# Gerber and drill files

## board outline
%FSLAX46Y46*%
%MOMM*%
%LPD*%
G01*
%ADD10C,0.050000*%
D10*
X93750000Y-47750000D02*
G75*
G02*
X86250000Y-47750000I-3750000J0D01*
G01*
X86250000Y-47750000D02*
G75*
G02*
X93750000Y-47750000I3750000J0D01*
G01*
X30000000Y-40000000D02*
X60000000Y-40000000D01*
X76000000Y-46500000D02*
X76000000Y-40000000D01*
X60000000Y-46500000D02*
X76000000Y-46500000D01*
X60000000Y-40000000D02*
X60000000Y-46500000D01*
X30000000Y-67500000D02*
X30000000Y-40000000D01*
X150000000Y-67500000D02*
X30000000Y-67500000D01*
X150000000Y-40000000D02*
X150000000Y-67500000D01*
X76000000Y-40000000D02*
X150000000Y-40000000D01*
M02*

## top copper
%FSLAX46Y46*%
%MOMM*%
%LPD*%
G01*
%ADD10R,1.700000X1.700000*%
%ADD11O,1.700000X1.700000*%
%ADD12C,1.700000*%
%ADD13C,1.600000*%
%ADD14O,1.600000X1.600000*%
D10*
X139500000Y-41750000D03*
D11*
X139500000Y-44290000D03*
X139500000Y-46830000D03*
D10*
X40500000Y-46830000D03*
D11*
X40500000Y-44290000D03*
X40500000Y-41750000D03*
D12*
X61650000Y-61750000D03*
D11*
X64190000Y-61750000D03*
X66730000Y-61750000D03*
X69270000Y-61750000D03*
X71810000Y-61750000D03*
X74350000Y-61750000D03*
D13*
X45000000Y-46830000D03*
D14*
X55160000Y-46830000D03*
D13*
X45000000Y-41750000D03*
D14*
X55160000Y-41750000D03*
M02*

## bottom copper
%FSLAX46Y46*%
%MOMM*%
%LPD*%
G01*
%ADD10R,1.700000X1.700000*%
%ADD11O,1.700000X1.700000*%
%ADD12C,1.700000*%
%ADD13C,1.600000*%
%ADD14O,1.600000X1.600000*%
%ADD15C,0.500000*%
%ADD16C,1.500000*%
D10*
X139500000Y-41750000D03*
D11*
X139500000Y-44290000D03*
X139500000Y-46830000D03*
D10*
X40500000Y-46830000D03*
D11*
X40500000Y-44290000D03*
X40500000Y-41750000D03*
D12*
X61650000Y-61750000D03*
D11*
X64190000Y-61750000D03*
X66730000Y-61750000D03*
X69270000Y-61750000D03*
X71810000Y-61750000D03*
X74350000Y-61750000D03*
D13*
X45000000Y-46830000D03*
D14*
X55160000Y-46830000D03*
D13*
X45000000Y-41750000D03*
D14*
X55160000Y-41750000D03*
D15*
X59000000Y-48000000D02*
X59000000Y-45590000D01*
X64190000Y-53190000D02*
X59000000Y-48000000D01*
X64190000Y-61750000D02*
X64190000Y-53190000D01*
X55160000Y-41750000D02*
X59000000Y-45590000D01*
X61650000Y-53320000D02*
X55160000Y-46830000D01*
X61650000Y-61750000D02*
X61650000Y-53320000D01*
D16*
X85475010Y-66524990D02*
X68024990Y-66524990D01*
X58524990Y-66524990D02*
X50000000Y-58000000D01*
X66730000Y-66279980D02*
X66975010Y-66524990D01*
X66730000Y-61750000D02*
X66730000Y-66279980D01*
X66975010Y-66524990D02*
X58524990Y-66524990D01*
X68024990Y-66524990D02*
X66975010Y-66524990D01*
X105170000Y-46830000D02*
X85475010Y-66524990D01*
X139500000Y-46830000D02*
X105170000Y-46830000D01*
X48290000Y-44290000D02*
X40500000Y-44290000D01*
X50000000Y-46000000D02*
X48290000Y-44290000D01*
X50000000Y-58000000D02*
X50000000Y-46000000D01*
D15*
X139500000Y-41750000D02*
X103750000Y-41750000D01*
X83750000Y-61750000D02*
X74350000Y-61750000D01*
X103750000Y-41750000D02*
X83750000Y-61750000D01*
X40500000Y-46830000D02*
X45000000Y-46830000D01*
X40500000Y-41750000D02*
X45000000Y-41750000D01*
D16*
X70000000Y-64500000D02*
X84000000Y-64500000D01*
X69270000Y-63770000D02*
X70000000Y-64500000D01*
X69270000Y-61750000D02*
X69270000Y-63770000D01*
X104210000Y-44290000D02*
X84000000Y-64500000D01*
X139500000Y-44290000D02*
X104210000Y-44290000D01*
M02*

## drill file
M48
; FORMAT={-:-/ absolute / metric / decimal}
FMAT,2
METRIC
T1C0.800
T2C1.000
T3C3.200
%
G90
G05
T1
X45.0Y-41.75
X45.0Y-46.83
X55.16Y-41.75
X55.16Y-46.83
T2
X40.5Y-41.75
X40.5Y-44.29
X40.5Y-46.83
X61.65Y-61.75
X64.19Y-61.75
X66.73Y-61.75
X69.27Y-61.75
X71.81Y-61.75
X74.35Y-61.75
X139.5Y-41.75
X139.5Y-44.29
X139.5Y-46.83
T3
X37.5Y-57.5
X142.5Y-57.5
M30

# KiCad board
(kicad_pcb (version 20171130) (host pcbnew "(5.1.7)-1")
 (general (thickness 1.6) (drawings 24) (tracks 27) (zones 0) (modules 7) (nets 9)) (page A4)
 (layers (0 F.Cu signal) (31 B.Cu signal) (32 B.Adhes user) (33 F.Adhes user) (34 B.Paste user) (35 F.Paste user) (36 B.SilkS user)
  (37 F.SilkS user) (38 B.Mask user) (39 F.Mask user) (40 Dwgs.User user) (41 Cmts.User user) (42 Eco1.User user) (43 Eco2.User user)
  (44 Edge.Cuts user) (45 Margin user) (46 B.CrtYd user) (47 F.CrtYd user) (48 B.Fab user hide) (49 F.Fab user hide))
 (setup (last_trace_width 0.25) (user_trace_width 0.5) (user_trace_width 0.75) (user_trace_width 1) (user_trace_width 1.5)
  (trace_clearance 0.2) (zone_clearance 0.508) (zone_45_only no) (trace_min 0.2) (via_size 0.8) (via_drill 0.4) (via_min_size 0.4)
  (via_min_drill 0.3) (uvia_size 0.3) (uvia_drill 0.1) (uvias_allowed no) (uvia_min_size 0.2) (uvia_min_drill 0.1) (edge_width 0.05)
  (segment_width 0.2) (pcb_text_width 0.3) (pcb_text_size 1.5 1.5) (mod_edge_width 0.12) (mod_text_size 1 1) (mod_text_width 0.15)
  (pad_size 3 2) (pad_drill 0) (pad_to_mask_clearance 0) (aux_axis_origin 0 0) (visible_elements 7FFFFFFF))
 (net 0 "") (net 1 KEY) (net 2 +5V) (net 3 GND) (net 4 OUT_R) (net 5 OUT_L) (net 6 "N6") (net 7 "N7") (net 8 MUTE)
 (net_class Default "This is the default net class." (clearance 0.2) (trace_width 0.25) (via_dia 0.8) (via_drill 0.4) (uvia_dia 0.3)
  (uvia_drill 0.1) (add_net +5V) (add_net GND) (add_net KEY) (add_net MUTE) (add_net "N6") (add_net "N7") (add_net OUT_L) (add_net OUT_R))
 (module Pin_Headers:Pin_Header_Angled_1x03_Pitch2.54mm (layer F.Cu) (at 139.5 41.75)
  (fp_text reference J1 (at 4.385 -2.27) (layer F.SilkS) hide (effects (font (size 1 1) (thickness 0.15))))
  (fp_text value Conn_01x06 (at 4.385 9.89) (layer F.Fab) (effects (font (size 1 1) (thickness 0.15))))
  (pad 1 thru_hole rect (at 0 0) (size 1.7 1.7) (drill 1) (layers *.Cu *.Mask) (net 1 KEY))
  (pad 2 thru_hole oval (at 0 2.54) (size 1.7 1.7) (drill 1) (layers *.Cu *.Mask) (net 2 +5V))
  (pad 3 thru_hole oval (at 0 5.08) (size 1.7 1.7) (drill 1) (layers *.Cu *.Mask) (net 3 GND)))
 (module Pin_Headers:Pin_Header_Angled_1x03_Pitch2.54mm (layer F.Cu) (at 40.5 46.83 180)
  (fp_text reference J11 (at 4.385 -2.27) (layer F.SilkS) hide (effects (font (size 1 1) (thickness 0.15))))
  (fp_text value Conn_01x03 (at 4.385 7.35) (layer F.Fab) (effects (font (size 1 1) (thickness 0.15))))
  (pad 1 thru_hole rect (at 0 0 180) (size 1.7 1.7) (drill 1) (layers *.Cu *.Mask) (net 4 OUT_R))
  (pad 2 thru_hole oval (at 0 2.54 180) (size 1.7 1.7) (drill 1) (layers *.Cu *.Mask) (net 3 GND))
  (pad 3 thru_hole oval (at 0 5.08 180) (size 1.7 1.7) (drill 1) (layers *.Cu *.Mask) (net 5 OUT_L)))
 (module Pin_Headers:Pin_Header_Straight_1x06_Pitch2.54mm (layer F.Cu) (at 61.65 61.75 90)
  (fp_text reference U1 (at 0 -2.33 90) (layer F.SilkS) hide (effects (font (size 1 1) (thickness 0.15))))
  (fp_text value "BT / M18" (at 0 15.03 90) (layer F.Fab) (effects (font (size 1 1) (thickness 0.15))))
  (pad 1 thru_hole circle (at 0 0 90) (size 1.7 1.7) (drill 1) (layers *.Cu *.Mask) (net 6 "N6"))
  (pad 2 thru_hole oval (at 0 2.54 90) (size 1.7 1.7) (drill 1) (layers *.Cu *.Mask) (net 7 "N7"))
  (pad 3 thru_hole oval (at 0 5.08 90) (size 1.7 1.7) (drill 1) (layers *.Cu *.Mask) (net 3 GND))
  (pad 4 thru_hole oval (at 0 7.62 90) (size 1.7 1.7) (drill 1) (layers *.Cu *.Mask) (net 2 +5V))
  (pad 5 thru_hole oval (at 0 10.16 90) (size 1.7 1.7) (drill 1) (layers *.Cu *.Mask) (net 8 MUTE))
  (pad 6 thru_hole oval (at 0 12.7 90) (size 1.7 1.7) (drill 1) (layers *.Cu *.Mask) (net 1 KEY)))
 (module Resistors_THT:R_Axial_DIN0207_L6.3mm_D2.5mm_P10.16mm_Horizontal (layer F.Cu) (at 45 46.83)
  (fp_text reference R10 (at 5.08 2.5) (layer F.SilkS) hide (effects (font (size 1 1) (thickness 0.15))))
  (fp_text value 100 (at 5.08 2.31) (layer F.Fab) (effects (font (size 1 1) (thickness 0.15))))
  (pad 1 thru_hole circle (at 0 0) (size 1.6 1.6) (drill 0.8) (layers *.Cu *.Mask) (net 4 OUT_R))
  (pad 2 thru_hole oval (at 10.16 0) (size 1.6 1.6) (drill 0.8) (layers *.Cu *.Mask) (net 6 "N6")))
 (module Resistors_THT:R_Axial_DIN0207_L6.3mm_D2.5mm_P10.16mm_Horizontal (layer F.Cu) (at 45 41.75)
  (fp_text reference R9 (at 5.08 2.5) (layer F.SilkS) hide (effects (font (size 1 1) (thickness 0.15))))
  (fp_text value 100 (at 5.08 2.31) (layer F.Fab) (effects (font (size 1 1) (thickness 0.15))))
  (pad 1 thru_hole circle (at 0 0) (size 1.6 1.6) (drill 0.8) (layers *.Cu *.Mask) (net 5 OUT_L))
  (pad 2 thru_hole oval (at 10.16 0) (size 1.6 1.6) (drill 0.8) (layers *.Cu *.Mask) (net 7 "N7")))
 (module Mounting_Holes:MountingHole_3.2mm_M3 (layer F.Cu) (at 142.5 57.5)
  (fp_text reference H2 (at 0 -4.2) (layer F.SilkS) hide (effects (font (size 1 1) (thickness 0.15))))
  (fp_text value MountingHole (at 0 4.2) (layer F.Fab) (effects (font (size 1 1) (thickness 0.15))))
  (pad 1 np_thru_hole circle (at 0 0) (size 3.2 3.2) (drill 3.2) (layers *.Cu *.Mask)))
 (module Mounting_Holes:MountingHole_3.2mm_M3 (layer F.Cu) (at 37.5 57.5)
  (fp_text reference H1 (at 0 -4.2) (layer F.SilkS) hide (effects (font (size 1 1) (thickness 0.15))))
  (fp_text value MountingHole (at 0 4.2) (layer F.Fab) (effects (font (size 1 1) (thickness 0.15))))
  (pad 1 np_thru_hole circle (at 0 0) (size 3.2 3.2) (drill 3.2) (layers *.Cu *.Mask)))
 (gr_circle (center 90 47.75) (end 93.75 47.75) (layer Edge.Cuts) (width 0.05))
 (gr_line (start 30 40) (end 60 40) (layer Edge.Cuts) (width 0.05))
 (gr_line (start 76 46.5) (end 76 40) (layer Edge.Cuts) (width 0.05))
 (gr_line (start 60 46.5) (end 76 46.5) (layer Edge.Cuts) (width 0.05))
 (gr_line (start 60 40) (end 60 46.5) (layer Edge.Cuts) (width 0.05))
 (gr_line (start 30 67.5) (end 30 40) (layer Edge.Cuts) (width 0.05))
 (gr_line (start 150 67.5) (end 30 67.5) (layer Edge.Cuts) (width 0.05))
 (gr_line (start 150 40) (end 150 67.5) (layer Edge.Cuts) (width 0.05))
 (gr_line (start 76 40) (end 150 40) (layer Edge.Cuts) (width 0.05))
 (segment (start 59 48) (end 59 45.59) (width 0.5) (layer B.Cu) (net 7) (status 1000000))
 (segment (start 64.19 53.19) (end 59 48) (width 0.5) (layer B.Cu) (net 7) (status 1000000))
 (segment (start 64.19 61.75) (end 64.19 53.19) (width 0.5) (layer B.Cu) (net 7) (status 1000000))
 (segment (start 55.16 41.75) (end 59 45.59) (width 0.5) (layer B.Cu) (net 7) (status 1000000))
 (segment (start 61.65 53.32) (end 55.16 46.83) (width 0.5) (layer B.Cu) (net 6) (status 1000000))
 (segment (start 61.65 61.75) (end 61.65 53.32) (width 0.5) (layer B.Cu) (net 6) (status 1000000))
 (segment (start 85.47501 66.52499) (end 68.02499 66.52499) (width 1.5) (layer B.Cu) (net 3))
 (segment (start 58.52499 66.52499) (end 50 58) (width 1.5) (layer B.Cu) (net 3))
 (segment (start 66.73 66.27998) (end 66.97501 66.52499) (width 1.5) (layer B.Cu) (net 3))
 (segment (start 66.73 61.75) (end 66.73 66.27998) (width 1.5) (layer B.Cu) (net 3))
 (segment (start 66.97501 66.52499) (end 58.52499 66.52499) (width 1.5) (layer B.Cu) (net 3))
 (segment (start 68.02499 66.52499) (end 66.97501 66.52499) (width 1.5) (layer B.Cu) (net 3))
 (segment (start 105.17 46.83) (end 85.47501 66.52499) (width 1.5) (layer B.Cu) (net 3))
 (segment (start 139.5 46.83) (end 105.17 46.83) (width 1.5) (layer B.Cu) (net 3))
 (segment (start 48.29 44.29) (end 40.5 44.29) (width 1.5) (layer B.Cu) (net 3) (status 1000000))
 (segment (start 50 46) (end 48.29 44.29) (width 1.5) (layer B.Cu) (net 3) (status 1000000))
 (segment (start 50 58) (end 50 46) (width 1.5) (layer B.Cu) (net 3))
 (segment (start 139.5 41.75) (end 103.75 41.75) (width 0.5) (layer B.Cu) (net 1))
 (segment (start 83.75 61.75) (end 74.35 61.75) (width 0.5) (layer B.Cu) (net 1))
 (segment (start 103.75 41.75) (end 83.75 61.75) (width 0.5) (layer B.Cu) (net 1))
 (segment (start 40.5 46.83) (end 45 46.83) (width 0.5) (layer B.Cu) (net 4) (status 1000000))
 (segment (start 40.5 41.75) (end 45 41.75) (width 0.5) (layer B.Cu) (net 5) (status 1000000))
 (segment (start 70 64.5) (end 84 64.5) (width 1.5) (layer B.Cu) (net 2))
 (segment (start 69.27 63.77) (end 70 64.5) (width 1.5) (layer B.Cu) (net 2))
 (segment (start 69.27 61.75) (end 69.27 63.77) (width 1.5) (layer B.Cu) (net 2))
 (segment (start 104.21 44.29) (end 84 64.5) (width 1.5) (layer B.Cu) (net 2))
 (segment (start 139.5 44.29) (end 104.21 44.29) (width 1.5) (layer B.Cu) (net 2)))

